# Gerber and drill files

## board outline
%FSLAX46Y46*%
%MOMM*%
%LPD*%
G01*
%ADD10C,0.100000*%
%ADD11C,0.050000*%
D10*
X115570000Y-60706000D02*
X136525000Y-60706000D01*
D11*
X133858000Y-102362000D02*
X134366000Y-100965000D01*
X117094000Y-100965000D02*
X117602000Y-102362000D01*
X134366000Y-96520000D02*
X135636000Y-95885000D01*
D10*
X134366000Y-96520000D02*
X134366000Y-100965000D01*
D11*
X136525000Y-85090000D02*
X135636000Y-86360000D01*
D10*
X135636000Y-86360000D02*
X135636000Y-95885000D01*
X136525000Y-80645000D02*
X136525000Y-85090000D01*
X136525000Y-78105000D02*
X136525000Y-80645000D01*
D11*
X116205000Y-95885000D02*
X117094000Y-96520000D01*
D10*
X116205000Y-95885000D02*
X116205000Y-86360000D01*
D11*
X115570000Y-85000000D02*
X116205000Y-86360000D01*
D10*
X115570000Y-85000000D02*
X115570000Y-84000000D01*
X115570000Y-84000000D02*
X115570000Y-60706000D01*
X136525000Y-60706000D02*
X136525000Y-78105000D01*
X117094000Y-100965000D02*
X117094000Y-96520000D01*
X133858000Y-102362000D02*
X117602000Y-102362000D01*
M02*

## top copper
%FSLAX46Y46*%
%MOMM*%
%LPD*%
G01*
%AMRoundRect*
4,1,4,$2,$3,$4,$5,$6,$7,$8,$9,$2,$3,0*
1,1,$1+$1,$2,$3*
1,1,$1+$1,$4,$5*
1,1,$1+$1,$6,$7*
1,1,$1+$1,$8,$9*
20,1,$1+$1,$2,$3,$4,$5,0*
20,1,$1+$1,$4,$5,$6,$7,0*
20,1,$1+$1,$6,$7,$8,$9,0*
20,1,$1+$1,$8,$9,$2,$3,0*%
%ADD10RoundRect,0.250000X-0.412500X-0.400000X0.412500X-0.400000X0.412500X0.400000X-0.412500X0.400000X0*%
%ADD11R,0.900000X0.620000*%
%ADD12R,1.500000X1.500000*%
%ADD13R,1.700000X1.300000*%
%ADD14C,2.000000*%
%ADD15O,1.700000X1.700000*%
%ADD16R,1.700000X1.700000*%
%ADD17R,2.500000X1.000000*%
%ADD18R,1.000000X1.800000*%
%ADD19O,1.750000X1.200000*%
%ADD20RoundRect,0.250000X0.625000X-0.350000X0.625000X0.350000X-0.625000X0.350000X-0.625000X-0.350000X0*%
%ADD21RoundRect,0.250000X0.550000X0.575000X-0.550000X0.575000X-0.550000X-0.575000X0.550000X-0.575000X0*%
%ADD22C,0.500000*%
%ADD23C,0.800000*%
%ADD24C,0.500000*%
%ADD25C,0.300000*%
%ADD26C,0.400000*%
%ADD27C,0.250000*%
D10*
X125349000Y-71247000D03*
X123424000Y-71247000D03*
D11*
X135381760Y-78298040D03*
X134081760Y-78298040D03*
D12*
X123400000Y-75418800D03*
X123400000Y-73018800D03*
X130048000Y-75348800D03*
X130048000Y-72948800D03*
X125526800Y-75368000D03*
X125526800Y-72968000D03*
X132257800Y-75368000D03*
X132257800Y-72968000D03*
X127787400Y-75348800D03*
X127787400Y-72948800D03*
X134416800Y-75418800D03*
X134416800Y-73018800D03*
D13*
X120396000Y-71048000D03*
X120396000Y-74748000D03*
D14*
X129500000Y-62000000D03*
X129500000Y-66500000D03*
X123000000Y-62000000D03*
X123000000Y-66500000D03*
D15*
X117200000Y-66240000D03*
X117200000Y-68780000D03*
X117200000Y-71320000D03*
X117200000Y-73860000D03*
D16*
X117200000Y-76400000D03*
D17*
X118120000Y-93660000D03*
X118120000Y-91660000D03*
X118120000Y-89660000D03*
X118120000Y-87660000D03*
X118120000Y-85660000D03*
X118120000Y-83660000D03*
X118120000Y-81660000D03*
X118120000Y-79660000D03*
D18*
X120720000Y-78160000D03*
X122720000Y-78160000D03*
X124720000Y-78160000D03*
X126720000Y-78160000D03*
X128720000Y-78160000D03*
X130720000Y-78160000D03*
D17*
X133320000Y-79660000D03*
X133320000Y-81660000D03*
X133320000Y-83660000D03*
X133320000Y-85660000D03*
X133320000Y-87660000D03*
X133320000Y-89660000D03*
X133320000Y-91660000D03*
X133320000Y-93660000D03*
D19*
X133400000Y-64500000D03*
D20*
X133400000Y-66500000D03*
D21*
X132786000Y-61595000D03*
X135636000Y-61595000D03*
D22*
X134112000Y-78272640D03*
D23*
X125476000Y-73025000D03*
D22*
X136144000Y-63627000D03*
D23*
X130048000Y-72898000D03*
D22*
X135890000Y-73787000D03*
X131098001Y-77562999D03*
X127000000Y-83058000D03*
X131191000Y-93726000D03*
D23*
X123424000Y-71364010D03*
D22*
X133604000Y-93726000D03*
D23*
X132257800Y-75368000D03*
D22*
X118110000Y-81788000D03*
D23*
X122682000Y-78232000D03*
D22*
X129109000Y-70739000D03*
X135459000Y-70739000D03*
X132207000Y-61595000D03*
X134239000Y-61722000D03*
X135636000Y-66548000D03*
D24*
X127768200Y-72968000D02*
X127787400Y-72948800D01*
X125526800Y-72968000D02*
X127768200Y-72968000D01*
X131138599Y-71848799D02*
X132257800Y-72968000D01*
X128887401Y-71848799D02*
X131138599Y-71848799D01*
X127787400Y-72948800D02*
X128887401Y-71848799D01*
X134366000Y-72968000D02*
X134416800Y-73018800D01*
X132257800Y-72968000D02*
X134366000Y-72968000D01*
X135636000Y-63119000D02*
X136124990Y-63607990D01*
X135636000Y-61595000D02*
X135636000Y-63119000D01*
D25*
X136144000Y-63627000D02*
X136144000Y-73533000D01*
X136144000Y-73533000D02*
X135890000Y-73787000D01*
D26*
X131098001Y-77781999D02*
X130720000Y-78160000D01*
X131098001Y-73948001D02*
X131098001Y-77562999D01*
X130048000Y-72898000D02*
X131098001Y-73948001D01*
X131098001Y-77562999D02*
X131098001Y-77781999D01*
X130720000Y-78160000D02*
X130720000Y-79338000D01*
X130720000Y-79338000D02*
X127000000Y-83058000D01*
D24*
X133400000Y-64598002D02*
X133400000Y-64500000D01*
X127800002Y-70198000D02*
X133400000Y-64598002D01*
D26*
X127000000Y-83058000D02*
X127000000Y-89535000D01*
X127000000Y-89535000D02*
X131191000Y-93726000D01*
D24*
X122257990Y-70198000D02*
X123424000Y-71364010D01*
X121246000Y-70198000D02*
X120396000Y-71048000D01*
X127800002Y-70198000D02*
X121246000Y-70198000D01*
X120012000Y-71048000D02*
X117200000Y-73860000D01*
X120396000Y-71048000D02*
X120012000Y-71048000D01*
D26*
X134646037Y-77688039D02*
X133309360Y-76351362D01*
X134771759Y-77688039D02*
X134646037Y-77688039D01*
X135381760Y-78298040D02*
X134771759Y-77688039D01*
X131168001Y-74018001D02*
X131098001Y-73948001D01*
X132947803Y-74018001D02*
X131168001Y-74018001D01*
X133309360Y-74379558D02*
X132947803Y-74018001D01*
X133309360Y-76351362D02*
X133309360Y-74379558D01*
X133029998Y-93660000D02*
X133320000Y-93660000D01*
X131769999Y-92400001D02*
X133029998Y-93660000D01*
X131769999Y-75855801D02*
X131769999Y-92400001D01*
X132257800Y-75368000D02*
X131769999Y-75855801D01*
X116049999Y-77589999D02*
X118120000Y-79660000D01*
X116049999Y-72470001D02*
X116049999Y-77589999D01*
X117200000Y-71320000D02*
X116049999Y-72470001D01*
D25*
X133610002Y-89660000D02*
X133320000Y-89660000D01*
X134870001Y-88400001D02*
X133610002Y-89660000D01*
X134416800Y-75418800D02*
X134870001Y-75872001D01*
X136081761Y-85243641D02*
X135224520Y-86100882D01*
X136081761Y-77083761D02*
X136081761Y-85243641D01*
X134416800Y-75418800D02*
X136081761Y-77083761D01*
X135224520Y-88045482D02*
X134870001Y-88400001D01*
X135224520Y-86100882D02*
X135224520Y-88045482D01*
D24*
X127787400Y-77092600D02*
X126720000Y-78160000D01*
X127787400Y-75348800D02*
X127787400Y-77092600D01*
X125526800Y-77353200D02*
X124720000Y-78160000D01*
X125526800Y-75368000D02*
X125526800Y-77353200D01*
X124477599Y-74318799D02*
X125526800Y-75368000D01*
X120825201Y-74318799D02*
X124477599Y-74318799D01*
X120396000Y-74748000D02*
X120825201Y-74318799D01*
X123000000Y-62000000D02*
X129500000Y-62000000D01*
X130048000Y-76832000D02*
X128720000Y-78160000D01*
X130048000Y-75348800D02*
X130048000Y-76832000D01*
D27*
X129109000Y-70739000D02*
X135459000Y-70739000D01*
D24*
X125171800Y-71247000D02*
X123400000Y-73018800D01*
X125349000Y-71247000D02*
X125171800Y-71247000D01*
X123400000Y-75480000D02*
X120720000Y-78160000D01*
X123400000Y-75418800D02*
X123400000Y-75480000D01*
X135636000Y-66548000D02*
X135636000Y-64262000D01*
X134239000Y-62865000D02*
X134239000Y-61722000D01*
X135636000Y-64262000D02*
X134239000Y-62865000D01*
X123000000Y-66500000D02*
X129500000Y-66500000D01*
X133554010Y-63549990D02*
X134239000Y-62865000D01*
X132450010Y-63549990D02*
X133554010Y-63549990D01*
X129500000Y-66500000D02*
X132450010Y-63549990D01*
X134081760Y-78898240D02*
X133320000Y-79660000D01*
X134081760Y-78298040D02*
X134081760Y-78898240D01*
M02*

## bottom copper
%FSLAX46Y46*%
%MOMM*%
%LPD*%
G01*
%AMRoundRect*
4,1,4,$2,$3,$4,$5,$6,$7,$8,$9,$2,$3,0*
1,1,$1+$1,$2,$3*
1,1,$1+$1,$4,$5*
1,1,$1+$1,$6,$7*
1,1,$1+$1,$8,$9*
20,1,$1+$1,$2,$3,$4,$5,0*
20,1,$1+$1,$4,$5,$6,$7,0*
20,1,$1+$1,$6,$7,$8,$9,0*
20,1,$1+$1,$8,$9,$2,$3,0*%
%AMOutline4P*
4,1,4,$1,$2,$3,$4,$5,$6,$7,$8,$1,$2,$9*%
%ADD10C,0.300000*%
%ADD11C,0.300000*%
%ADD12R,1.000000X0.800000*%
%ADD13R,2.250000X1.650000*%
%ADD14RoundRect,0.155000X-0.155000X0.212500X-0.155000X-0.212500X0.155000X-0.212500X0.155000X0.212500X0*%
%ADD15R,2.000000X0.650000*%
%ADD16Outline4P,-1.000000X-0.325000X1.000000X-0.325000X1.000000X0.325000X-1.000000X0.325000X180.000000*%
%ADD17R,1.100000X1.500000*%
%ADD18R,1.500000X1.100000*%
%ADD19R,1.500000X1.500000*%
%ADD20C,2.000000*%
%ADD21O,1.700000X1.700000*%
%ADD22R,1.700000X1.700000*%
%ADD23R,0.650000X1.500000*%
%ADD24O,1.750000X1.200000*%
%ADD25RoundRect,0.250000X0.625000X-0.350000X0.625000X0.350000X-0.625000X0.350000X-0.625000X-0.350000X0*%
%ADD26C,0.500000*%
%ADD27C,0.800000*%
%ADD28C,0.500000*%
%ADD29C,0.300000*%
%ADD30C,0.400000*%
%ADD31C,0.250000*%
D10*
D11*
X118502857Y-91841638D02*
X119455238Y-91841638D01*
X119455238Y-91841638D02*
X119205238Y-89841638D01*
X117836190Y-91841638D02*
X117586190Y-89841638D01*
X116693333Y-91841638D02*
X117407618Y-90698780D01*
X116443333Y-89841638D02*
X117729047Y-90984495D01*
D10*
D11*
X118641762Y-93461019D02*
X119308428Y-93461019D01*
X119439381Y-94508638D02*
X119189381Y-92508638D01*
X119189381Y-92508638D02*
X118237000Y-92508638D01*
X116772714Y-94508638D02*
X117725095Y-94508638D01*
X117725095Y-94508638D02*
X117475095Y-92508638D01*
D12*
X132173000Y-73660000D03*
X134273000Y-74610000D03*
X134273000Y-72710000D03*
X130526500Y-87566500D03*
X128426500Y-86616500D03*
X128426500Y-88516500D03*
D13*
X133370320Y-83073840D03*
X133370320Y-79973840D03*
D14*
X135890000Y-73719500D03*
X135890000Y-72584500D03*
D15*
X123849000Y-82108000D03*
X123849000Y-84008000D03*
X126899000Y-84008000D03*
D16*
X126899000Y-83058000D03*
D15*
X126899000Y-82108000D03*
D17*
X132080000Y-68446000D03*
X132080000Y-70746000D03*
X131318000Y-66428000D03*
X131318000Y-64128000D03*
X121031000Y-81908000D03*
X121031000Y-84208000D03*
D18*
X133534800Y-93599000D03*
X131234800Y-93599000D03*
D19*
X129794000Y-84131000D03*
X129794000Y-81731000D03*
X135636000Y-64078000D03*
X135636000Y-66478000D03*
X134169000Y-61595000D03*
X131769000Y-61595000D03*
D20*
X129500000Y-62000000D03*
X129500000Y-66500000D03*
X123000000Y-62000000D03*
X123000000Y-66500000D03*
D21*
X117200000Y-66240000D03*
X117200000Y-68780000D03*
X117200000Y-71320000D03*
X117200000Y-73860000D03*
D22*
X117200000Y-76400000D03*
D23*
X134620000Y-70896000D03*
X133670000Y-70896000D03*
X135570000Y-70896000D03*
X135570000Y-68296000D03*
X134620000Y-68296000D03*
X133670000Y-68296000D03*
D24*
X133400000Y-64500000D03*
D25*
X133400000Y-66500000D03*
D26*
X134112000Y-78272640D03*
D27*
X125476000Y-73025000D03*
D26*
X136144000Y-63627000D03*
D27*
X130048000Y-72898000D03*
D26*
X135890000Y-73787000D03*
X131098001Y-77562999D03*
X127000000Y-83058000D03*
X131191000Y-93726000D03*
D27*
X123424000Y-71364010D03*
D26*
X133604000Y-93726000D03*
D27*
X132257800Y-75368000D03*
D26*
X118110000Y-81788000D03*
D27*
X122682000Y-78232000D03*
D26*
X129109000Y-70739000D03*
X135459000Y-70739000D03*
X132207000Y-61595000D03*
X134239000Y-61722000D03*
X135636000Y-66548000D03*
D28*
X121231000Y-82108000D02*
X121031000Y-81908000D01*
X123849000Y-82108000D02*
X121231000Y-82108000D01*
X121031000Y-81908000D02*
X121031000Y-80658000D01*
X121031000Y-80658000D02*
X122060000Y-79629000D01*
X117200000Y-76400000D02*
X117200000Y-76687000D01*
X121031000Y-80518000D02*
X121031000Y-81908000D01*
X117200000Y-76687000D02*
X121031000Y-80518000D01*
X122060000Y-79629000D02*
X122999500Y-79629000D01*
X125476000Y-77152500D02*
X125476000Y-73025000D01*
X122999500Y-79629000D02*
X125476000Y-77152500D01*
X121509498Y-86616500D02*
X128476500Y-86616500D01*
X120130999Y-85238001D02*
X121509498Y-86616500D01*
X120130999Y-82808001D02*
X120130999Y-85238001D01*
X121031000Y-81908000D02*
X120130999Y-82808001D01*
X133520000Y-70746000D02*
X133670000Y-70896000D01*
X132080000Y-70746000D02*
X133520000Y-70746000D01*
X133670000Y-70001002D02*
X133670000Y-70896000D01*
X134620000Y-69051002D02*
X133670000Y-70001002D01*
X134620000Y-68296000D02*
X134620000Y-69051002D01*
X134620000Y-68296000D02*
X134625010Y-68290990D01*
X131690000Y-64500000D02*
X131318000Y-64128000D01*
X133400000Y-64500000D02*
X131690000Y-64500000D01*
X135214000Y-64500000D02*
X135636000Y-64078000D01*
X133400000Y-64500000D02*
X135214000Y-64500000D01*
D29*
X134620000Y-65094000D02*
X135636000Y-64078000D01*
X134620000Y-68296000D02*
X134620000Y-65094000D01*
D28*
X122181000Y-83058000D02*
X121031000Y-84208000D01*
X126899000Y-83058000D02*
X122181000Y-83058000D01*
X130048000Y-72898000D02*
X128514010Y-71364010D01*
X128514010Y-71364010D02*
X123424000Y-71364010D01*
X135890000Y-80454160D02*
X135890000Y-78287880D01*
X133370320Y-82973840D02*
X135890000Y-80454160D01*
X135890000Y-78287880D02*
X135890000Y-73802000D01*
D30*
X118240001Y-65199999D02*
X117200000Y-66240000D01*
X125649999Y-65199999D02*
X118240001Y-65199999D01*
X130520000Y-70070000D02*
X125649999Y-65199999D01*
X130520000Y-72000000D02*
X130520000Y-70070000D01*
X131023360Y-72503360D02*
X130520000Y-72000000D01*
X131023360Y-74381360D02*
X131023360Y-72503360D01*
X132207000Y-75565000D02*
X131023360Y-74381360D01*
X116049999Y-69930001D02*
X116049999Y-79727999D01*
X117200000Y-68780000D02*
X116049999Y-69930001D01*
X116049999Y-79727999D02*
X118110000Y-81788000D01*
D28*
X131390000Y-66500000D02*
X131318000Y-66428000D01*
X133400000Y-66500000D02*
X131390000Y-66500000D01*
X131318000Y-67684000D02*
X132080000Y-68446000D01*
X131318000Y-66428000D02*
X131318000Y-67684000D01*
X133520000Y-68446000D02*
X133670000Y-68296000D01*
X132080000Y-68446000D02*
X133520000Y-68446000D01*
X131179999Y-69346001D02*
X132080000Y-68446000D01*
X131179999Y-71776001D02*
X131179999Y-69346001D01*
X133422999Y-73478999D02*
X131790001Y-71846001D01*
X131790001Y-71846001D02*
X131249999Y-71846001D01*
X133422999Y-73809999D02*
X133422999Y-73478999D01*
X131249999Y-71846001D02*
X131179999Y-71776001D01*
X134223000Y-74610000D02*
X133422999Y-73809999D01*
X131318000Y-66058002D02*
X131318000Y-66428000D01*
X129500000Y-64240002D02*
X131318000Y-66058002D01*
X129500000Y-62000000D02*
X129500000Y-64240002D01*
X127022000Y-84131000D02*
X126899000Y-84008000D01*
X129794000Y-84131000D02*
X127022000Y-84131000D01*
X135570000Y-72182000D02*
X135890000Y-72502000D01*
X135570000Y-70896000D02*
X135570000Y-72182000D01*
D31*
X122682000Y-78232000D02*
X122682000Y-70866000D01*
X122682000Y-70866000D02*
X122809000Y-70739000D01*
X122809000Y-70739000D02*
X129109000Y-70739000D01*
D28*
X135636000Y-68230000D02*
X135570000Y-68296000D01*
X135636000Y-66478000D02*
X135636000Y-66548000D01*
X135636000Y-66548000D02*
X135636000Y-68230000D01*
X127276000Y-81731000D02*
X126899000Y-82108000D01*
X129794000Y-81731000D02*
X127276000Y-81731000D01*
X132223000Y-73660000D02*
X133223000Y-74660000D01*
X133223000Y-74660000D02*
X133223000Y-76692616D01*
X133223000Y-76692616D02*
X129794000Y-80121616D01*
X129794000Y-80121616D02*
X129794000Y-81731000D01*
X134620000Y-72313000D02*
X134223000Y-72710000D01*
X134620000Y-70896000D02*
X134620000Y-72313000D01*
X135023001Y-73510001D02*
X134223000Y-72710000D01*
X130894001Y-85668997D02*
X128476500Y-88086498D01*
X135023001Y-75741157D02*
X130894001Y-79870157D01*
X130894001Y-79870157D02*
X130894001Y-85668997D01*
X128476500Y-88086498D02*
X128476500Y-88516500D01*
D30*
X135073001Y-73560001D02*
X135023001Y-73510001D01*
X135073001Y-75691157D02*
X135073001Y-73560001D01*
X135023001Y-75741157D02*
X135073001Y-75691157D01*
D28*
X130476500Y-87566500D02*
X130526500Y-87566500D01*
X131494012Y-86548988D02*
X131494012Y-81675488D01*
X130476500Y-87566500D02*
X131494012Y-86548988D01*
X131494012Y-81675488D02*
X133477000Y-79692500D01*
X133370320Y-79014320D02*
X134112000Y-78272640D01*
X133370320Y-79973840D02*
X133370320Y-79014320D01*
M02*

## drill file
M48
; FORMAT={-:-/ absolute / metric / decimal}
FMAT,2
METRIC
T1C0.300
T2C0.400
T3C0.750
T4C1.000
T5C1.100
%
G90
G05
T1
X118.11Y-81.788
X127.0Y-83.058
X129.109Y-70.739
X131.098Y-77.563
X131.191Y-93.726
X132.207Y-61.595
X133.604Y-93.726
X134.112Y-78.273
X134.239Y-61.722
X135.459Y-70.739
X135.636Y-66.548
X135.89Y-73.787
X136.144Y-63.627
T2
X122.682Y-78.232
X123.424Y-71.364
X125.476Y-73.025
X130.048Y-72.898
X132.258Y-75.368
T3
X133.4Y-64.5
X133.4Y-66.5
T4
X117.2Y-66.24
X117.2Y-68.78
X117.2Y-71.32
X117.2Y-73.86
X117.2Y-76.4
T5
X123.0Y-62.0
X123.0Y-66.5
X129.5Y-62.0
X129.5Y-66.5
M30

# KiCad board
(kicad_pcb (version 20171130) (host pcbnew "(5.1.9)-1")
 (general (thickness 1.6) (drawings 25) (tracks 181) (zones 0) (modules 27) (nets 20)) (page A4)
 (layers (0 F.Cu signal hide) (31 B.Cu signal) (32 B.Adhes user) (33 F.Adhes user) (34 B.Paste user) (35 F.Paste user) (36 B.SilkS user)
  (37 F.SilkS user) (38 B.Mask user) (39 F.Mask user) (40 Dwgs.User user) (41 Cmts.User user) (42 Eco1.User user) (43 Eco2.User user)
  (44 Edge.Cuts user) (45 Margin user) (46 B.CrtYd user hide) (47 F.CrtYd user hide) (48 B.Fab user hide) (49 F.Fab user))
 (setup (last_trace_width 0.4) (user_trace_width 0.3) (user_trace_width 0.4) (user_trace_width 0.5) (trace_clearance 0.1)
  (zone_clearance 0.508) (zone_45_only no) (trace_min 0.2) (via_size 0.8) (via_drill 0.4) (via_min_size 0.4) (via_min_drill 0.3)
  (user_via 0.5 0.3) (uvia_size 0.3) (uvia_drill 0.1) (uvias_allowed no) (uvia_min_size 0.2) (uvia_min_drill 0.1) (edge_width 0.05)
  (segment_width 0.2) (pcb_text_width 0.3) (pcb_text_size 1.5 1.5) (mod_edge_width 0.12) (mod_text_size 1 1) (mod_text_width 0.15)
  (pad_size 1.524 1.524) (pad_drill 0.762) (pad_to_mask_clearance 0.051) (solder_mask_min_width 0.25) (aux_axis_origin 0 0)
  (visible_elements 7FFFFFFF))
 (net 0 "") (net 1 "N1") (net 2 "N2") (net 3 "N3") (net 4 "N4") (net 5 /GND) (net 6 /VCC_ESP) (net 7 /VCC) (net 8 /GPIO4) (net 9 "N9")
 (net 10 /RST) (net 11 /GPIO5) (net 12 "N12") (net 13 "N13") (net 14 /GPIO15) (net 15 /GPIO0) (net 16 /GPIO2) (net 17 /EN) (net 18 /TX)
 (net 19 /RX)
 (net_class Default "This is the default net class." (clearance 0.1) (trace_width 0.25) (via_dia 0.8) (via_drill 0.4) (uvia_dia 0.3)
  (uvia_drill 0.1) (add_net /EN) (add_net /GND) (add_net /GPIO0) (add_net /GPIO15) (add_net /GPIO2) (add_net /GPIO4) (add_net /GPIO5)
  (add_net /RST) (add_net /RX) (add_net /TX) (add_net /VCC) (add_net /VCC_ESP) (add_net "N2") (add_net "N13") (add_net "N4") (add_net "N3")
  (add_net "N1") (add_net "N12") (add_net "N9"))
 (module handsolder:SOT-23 (layer B.Cu) (at 133.223 73.66 180)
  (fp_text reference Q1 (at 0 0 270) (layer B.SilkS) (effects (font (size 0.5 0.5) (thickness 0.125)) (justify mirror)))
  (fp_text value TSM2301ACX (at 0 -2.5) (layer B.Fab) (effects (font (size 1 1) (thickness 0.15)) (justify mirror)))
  (pad 3 smd rect (at 1.05 0 180) (size 1 0.8) (layers B.Cu B.Paste B.Mask) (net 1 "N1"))
  (pad 2 smd rect (at -1.05 -0.95 180) (size 1 0.8) (layers B.Cu B.Paste B.Mask) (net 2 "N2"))
  (pad 1 smd rect (at -1.05 0.95 180) (size 1 0.8) (layers B.Cu B.Paste B.Mask) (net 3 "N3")))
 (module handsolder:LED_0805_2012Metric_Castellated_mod (layer F.Cu) (at 124.3865 71.247)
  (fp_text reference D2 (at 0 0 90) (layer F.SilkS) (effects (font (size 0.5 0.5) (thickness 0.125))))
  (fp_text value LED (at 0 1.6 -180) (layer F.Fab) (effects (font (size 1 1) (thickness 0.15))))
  (pad 2 smd roundrect (at 0.9625 0) (size 1.325 1.3) (layers F.Cu F.Paste F.Mask) (roundrect_rratio 0.1923076923076923) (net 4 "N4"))
  (pad 1 smd roundrect (at -0.9625 0) (size 1.325 1.3) (layers F.Cu F.Paste F.Mask) (roundrect_rratio 0.1923076923076923) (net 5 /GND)))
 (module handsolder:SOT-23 (layer B.Cu) (at 129.4765 87.5665)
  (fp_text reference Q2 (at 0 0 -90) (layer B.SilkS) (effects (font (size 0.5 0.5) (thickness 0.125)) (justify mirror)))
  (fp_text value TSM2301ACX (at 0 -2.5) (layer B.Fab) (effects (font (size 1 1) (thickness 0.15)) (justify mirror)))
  (pad 3 smd rect (at 1.05 0) (size 1 0.8) (layers B.Cu B.Paste B.Mask) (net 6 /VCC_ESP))
  (pad 2 smd rect (at -1.05 -0.95) (size 1 0.8) (layers B.Cu B.Paste B.Mask) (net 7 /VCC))
  (pad 1 smd rect (at -1.05 0.95) (size 1 0.8) (layers B.Cu B.Paste B.Mask) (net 3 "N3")))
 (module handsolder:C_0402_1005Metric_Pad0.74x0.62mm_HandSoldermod (layer F.Cu) (at 134.73176 78.29804)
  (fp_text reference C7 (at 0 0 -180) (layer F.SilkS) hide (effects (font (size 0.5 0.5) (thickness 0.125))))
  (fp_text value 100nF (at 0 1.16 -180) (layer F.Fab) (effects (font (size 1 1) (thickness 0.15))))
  (pad 2 smd rect (at 0.65 0) (size 0.9 0.62) (layers F.Cu F.Paste F.Mask) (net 5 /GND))
  (pad 1 smd rect (at -0.65 0) (size 0.9 0.62) (layers F.Cu F.Paste F.Mask) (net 6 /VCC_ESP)))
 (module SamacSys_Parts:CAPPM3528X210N (layer B.Cu) (at 133.37032 81.52384 270)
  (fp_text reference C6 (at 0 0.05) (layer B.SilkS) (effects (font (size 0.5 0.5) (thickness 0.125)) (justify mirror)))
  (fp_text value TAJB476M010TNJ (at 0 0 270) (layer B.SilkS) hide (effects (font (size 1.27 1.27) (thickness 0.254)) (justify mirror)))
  (pad 2 smd rect (at 1.55 0 270) (size 1.65 2.25) (layers B.Cu B.Paste B.Mask) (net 5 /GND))
  (pad 1 smd rect (at -1.55 0 270) (size 1.65 2.25) (layers B.Cu B.Paste B.Mask) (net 6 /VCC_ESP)))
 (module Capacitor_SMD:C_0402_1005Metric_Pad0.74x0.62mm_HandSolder (layer B.Cu) (at 135.89 73.152 270)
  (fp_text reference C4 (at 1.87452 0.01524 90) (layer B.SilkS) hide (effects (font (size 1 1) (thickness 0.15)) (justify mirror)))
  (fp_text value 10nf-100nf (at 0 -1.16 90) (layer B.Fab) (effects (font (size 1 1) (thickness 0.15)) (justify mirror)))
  (pad 2 smd roundrect (at 0.5675 0 270) (size 0.735 0.62) (layers B.Cu B.Paste B.Mask) (roundrect_rratio 0.25) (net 5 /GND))
  (pad 1 smd roundrect (at -0.5675 0 270) (size 0.735 0.62) (layers B.Cu B.Paste B.Mask) (roundrect_rratio 0.25) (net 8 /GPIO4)))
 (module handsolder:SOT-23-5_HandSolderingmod (layer B.Cu) (at 125.349 83.058 180)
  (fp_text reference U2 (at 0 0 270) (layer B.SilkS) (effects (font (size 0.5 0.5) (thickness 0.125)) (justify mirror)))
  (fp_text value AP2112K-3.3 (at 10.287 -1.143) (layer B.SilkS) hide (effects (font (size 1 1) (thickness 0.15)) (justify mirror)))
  (pad 5 smd rect (at 1.5 0.95 180) (size 2 0.65) (layers B.Cu B.Paste B.Mask) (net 7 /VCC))
  (pad 4 smd rect (at 1.5 -0.95 180) (size 2 0.65) (layers B.Cu B.Paste B.Mask))
  (pad 3 smd rect (at -1.55 -0.95 180) (size 2 0.65) (layers B.Cu B.Paste B.Mask) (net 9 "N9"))
  (pad 2 smd trapezoid (at -1.55 0 180) (size 2 0.65) (layers B.Cu B.Paste B.Mask) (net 5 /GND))
  (pad 1 smd rect (at -1.55 0.95 180) (size 2 0.65) (layers B.Cu B.Paste B.Mask) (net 1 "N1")))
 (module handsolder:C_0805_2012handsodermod (layer B.Cu) (at 132.08 69.596 90)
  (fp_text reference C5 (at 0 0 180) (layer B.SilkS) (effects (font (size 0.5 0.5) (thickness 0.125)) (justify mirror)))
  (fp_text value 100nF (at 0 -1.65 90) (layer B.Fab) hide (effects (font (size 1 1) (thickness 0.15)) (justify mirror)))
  (pad 2 smd rect (at 1.15 0 90) (size 1.5 1.1) (layers B.Cu B.Paste B.Mask) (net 2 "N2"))
  (pad 1 smd rect (at -1.15 0 90) (size 1.5 1.1) (layers B.Cu B.Paste B.Mask) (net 5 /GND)))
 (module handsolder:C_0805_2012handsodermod (layer B.Cu) (at 131.318 65.278 270)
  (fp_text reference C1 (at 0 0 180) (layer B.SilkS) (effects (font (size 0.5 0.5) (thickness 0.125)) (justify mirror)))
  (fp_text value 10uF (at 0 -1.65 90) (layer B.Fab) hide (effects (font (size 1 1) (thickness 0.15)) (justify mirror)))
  (pad 2 smd rect (at 1.15 0 270) (size 1.5 1.1) (layers B.Cu B.Paste B.Mask) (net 2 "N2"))
  (pad 1 smd rect (at -1.15 0 270) (size 1.5 1.1) (layers B.Cu B.Paste B.Mask) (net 5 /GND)))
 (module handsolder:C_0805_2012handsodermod (layer B.Cu) (at 121.031 83.058 90)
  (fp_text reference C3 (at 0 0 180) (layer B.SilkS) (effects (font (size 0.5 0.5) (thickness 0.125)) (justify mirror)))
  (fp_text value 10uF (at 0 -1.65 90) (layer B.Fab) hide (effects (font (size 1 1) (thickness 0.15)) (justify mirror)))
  (pad 2 smd rect (at 1.15 0 90) (size 1.5 1.1) (layers B.Cu B.Paste B.Mask) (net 7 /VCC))
  (pad 1 smd rect (at -1.15 0 90) (size 1.5 1.1) (layers B.Cu B.Paste B.Mask) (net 5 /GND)))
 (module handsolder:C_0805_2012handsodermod (layer B.Cu) (at 132.3848 93.599)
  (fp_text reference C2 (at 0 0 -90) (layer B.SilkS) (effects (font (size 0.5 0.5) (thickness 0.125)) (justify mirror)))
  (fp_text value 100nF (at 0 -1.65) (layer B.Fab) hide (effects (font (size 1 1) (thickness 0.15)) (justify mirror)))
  (pad 2 smd rect (at 1.15 0) (size 1.5 1.1) (layers B.Cu B.Paste B.Mask) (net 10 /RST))
  (pad 1 smd rect (at -1.15 0) (size 1.5 1.1) (layers B.Cu B.Paste B.Mask) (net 5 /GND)))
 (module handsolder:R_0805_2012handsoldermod (layer F.Cu) (at 123.4 74.2188 270)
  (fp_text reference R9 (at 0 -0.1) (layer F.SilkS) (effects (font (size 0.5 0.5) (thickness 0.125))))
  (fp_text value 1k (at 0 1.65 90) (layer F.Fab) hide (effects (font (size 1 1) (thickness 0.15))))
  (pad 2 smd rect (at 1.2 0 270) (size 1.5 1.5) (layers F.Cu F.Paste F.Mask) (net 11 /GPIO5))
  (pad 1 smd rect (at -1.2 0 270) (size 1.5 1.5) (layers F.Cu F.Paste F.Mask) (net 4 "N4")))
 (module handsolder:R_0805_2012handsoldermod (layer B.Cu) (at 129.794 82.931 270)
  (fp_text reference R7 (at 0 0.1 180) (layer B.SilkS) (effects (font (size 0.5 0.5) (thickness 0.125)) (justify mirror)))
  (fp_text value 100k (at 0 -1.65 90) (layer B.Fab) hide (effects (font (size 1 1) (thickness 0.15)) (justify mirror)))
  (pad 2 smd rect (at 1.2 0 270) (size 1.5 1.5) (layers B.Cu B.Paste B.Mask) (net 9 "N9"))
  (pad 1 smd rect (at -1.2 0 270) (size 1.5 1.5) (layers B.Cu B.Paste B.Mask) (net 1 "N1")))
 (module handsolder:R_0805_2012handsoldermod (layer B.Cu) (at 135.636 65.278 90)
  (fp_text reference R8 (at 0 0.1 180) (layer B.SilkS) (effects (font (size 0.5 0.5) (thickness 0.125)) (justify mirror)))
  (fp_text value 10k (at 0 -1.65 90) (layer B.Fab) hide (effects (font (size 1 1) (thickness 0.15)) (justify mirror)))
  (pad 2 smd rect (at 1.2 0 90) (size 1.5 1.5) (layers B.Cu B.Paste B.Mask) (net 5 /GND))
  (pad 1 smd rect (at -1.2 0 90) (size 1.5 1.5) (layers B.Cu B.Paste B.Mask) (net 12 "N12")))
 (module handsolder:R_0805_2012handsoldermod (layer B.Cu) (at 132.969 61.595)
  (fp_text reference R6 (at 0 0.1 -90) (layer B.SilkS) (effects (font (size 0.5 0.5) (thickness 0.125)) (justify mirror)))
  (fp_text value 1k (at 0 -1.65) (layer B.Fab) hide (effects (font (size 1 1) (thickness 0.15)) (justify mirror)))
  (pad 2 smd rect (at 1.2 0) (size 1.5 1.5) (layers B.Cu B.Paste B.Mask) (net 12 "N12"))
  (pad 1 smd rect (at -1.2 0) (size 1.5 1.5) (layers B.Cu B.Paste B.Mask) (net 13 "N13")))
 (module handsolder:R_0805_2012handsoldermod (layer F.Cu) (at 130.048 74.1488 270)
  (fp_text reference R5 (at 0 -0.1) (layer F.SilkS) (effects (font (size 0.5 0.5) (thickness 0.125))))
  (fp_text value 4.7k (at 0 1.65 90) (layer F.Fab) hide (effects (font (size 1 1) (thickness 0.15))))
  (pad 2 smd rect (at 1.2 0 270) (size 1.5 1.5) (layers F.Cu F.Paste F.Mask) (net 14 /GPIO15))
  (pad 1 smd rect (at -1.2 0 270) (size 1.5 1.5) (layers F.Cu F.Paste F.Mask) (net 5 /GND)))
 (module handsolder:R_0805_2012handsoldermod (layer F.Cu) (at 125.5268 74.168 270)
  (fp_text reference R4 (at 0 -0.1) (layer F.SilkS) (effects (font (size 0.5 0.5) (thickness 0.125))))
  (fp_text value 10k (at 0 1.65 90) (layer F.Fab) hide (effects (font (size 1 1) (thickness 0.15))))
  (pad 2 smd rect (at 1.2 0 270) (size 1.5 1.5) (layers F.Cu F.Paste F.Mask) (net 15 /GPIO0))
  (pad 1 smd rect (at -1.2 0 270) (size 1.5 1.5) (layers F.Cu F.Paste F.Mask) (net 7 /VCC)))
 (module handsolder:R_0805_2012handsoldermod (layer F.Cu) (at 132.2578 74.168 270)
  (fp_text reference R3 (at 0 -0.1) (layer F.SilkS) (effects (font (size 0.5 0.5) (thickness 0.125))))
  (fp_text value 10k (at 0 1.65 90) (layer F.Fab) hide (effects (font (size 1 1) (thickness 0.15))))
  (pad 2 smd rect (at 1.2 0 270) (size 1.5 1.5) (layers F.Cu F.Paste F.Mask) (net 10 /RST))
  (pad 1 smd rect (at -1.2 0 270) (size 1.5 1.5) (layers F.Cu F.Paste F.Mask) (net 7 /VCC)))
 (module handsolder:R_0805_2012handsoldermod (layer F.Cu) (at 127.7874 74.1488 270)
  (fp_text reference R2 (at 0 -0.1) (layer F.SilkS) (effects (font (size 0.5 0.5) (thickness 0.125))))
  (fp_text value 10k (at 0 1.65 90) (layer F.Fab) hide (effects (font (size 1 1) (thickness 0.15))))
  (pad 2 smd rect (at 1.2 0 270) (size 1.5 1.5) (layers F.Cu F.Paste F.Mask) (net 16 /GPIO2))
  (pad 1 smd rect (at -1.2 0 270) (size 1.5 1.5) (layers F.Cu F.Paste F.Mask) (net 7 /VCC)))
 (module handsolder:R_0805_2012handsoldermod (layer F.Cu) (at 134.4168 74.2188 270)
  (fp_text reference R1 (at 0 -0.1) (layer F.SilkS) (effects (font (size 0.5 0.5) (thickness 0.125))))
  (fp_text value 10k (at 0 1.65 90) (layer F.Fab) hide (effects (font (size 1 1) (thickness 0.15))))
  (pad 2 smd rect (at 1.2 0 270) (size 1.5 1.5) (layers F.Cu F.Paste F.Mask) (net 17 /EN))
  (pad 1 smd rect (at -1.2 0 270) (size 1.5 1.5) (layers F.Cu F.Paste F.Mask) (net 7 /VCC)))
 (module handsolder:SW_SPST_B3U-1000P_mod (layer F.Cu) (at 120.396 72.898 90)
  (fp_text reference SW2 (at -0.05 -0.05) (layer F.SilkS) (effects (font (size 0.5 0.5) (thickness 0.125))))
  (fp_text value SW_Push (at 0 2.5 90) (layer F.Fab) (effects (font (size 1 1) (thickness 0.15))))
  (pad 2 smd rect (at 1.85 0 90) (size 1.3 1.7) (layers F.Cu F.Paste F.Mask) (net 5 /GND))
  (pad 1 smd rect (at -1.85 0 90) (size 1.3 1.7) (layers F.Cu F.Paste F.Mask) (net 15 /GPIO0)))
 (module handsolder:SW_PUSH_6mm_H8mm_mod (layer F.Cu) (at 123 62)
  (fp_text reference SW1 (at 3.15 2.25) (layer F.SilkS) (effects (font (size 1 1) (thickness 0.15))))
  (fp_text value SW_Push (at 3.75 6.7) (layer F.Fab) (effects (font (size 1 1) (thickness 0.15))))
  (pad 1 thru_hole circle (at 6.5 0 90) (size 2 2) (drill 1.1) (layers *.Cu *.Mask) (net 2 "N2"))
  (pad 2 thru_hole circle (at 6.5 4.5 90) (size 2 2) (drill 1.1) (layers *.Cu *.Mask) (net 12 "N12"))
  (pad 1 thru_hole circle (at 0 0 90) (size 2 2) (drill 1.1) (layers *.Cu *.Mask) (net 2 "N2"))
  (pad 2 thru_hole circle (at 0 4.5 90) (size 2 2) (drill 1.1) (layers *.Cu *.Mask) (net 12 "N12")))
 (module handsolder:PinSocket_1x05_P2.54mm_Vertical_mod (layer F.Cu) (at 117.2 76.4 180)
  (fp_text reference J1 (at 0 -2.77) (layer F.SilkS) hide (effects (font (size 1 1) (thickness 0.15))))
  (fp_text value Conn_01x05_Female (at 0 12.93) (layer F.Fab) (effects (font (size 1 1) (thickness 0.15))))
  (pad 5 thru_hole oval (at 0 10.16 180) (size 1.7 1.7) (drill 1) (layers *.Cu *.Mask) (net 10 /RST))
  (pad 4 thru_hole oval (at 0 7.62 180) (size 1.7 1.7) (drill 1) (layers *.Cu *.Mask) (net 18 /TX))
  (pad 3 thru_hole oval (at 0 5.08 180) (size 1.7 1.7) (drill 1) (layers *.Cu *.Mask) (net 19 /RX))
  (pad 2 thru_hole oval (at 0 2.54 180) (size 1.7 1.7) (drill 1) (layers *.Cu *.Mask) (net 5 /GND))
  (pad 1 thru_hole rect (at 0 0 180) (size 1.7 1.7) (drill 1) (layers *.Cu *.Mask) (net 7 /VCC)))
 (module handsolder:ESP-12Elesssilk (layer F.Cu) (at 125.72 90.16 180)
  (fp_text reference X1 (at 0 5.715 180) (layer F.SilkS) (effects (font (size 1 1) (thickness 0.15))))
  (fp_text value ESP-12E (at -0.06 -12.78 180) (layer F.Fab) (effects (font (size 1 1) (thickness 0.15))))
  (pad 22 smd rect (at 7.6 -3.5 180) (size 2.5 1) (layers F.Cu F.Paste F.Mask))
  (pad 21 smd rect (at 7.6 -1.5 180) (size 2.5 1) (layers F.Cu F.Paste F.Mask))
  (pad 20 smd rect (at 7.6 0.5 180) (size 2.5 1) (layers F.Cu F.Paste F.Mask))
  (pad 19 smd rect (at 7.6 2.5 180) (size 2.5 1) (layers F.Cu F.Paste F.Mask))
  (pad 18 smd rect (at 7.6 4.5 180) (size 2.5 1) (layers F.Cu F.Paste F.Mask))
  (pad 17 smd rect (at 7.6 6.5 180) (size 2.5 1) (layers F.Cu F.Paste F.Mask))
  (pad 16 smd rect (at 7.6 8.5 180) (size 2.5 1) (layers F.Cu F.Paste F.Mask) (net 18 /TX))
  (pad 15 smd rect (at 7.6 10.5 180) (size 2.5 1) (layers F.Cu F.Paste F.Mask) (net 19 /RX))
  (pad 14 smd rect (at 5 12 180) (size 1 1.8) (layers F.Cu F.Paste F.Mask) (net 11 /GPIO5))
  (pad 13 smd rect (at 3 12 180) (size 1 1.8) (layers F.Cu F.Paste F.Mask) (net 8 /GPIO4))
  (pad 12 smd rect (at 1 12 180) (size 1 1.8) (layers F.Cu F.Paste F.Mask) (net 15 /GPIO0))
  (pad 11 smd rect (at -1 12 180) (size 1 1.8) (layers F.Cu F.Paste F.Mask) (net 16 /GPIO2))
  (pad 10 smd rect (at -3 12 180) (size 1 1.8) (layers F.Cu F.Paste F.Mask) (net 14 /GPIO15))
  (pad 9 smd rect (at -5 12 180) (size 1 1.8) (layers F.Cu F.Paste F.Mask) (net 5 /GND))
  (pad 8 smd rect (at -7.6 10.5 180) (size 2.5 1) (layers F.Cu F.Paste F.Mask) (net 6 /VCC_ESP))
  (pad 7 smd rect (at -7.6 8.5 180) (size 2.5 1) (layers F.Cu F.Paste F.Mask))
  (pad 6 smd rect (at -7.6 6.5 180) (size 2.5 1) (layers F.Cu F.Paste F.Mask))
  (pad 5 smd rect (at -7.6 4.5 180) (size 2.5 1) (layers F.Cu F.Paste F.Mask))
  (pad 4 smd rect (at -7.6 2.5 180) (size 2.5 1) (layers F.Cu F.Paste F.Mask))
  (pad 3 smd rect (at -7.6 0.5 180) (size 2.5 1) (layers F.Cu F.Paste F.Mask) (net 17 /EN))
  (pad 2 smd rect (at -7.6 -1.5 180) (size 2.5 1) (layers F.Cu F.Paste F.Mask))
  (pad 1 smd rect (at -7.6 -3.5 180) (size 2.5 1) (layers F.Cu F.Paste F.Mask) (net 10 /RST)))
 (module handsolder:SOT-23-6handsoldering (layer B.Cu) (at 134.62 69.596 270)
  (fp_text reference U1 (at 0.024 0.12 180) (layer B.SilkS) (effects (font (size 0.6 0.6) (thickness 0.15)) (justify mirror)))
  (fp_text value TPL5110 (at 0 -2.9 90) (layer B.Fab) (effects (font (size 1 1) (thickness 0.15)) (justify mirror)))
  (pad 5 smd rect (at 1.3 0 270) (size 1.5 0.65) (layers B.Cu B.Paste B.Mask) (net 3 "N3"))
  (pad 6 smd rect (at 1.3 0.95 270) (size 1.5 0.65) (layers B.Cu B.Paste B.Mask) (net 5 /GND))
  (pad 4 smd rect (at 1.3 -0.95 270) (size 1.5 0.65) (layers B.Cu B.Paste B.Mask) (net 8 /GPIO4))
  (pad 3 smd rect (at -1.3 -0.95 270) (size 1.5 0.65) (layers B.Cu B.Paste B.Mask) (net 12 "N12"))
  (pad 2 smd rect (at -1.3 0 270) (size 1.5 0.65) (layers B.Cu B.Paste B.Mask) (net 5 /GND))
  (pad 1 smd rect (at -1.3 0.95 270) (size 1.5 0.65) (layers B.Cu B.Paste B.Mask) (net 2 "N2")))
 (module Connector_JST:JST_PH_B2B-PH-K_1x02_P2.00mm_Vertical (layer F.Cu) (at 133.4 66.5 90)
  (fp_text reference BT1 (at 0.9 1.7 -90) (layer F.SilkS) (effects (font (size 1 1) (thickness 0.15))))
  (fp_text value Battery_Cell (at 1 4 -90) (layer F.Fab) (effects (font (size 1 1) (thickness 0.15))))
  (pad 2 thru_hole oval (at 2 0 90) (size 1.2 1.75) (drill 0.75) (layers *.Cu *.Mask) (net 5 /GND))
  (pad 1 thru_hole roundrect (at 0 0 90) (size 1.2 1.75) (drill 0.75) (layers *.Cu *.Mask) (roundrect_rratio 0.208333) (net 2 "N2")))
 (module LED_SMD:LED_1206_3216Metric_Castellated (layer F.Cu) (at 134.211 61.595 180)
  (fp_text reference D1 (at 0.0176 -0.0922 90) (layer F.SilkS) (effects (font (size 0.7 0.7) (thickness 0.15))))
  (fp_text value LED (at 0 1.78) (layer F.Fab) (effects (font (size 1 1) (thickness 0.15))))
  (pad 2 smd roundrect (at 1.425 0 180) (size 1.6 1.65) (layers F.Cu F.Paste F.Mask) (roundrect_rratio 0.15625) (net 13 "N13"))
  (pad 1 smd roundrect (at -1.425 0 180) (size 1.6 1.65) (layers F.Cu F.Paste F.Mask) (roundrect_rratio 0.15625) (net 5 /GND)))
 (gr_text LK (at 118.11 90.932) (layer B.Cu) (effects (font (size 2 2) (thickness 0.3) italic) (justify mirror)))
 (gr_line (start 115.57 60.706) (end 136.525 60.706) (layer Edge.Cuts) (width 0.1))
 (gr_line (start 133.858 102.362) (end 134.366 100.965) (layer Edge.Cuts) (width 0.05))
 (gr_line (start 117.094 100.965) (end 117.602 102.362) (layer Edge.Cuts) (width 0.05))
 (gr_line (start 134.366 96.52) (end 135.636 95.885) (layer Edge.Cuts) (width 0.05))
 (gr_line (start 134.366 96.52) (end 134.366 100.965) (layer Edge.Cuts) (width 0.1))
 (gr_line (start 136.525 85.09) (end 135.636 86.36) (layer Edge.Cuts) (width 0.05))
 (gr_line (start 135.636 86.36) (end 135.636 95.885) (layer Edge.Cuts) (width 0.1))
 (gr_line (start 136.525 80.645) (end 136.525 85.09) (layer Edge.Cuts) (width 0.1))
 (gr_line (start 136.525 78.105) (end 136.525 80.645) (layer Edge.Cuts) (width 0.1))
 (gr_line (start 116.205 95.885) (end 117.094 96.52) (layer Edge.Cuts) (width 0.05))
 (gr_line (start 116.205 95.885) (end 116.205 86.36) (layer Edge.Cuts) (width 0.1))
 (gr_line (start 115.57 85) (end 116.205 86.36) (layer Edge.Cuts) (width 0.05))
 (gr_line (start 115.57 85) (end 115.57 84) (layer Edge.Cuts) (width 0.1))
 (gr_line (start 115.57 84) (end 115.57 60.706) (layer Edge.Cuts) (width 0.1))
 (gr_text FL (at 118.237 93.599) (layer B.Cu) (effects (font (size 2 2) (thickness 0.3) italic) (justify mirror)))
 (gr_line (start 136.525 60.706) (end 136.525 78.105) (layer Edge.Cuts) (width 0.1))
 (gr_line (start 117.094 100.965) (end 117.094 96.52) (layer Edge.Cuts) (width 0.1))
 (gr_line (start 133.858 102.362) (end 117.602 102.362) (layer Edge.Cuts) (width 0.1))
 (via (at 134.112 78.27264) (size 0.5) (drill 0.3) (layers F.Cu B.Cu) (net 6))
 (via (at 125.476 73.025) (size 0.8) (drill 0.4) (layers F.Cu B.Cu) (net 7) (status 30))
 (segment (start 121.231 82.108) (end 121.031 81.908) (width 0.5) (layer B.Cu) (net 7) (status 30))
 (segment (start 123.849 82.108) (end 121.231 82.108) (width 0.5) (layer B.Cu) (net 7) (status 30))
 (segment (start 121.031 81.908) (end 121.031 80.658) (width 0.5) (layer B.Cu) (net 7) (status 10))
 (segment (start 121.031 80.658) (end 122.06 79.629) (width 0.5) (layer B.Cu) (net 7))
 (segment (start 127.7682 72.968) (end 127.7874 72.9488) (width 0.5) (layer F.Cu) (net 7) (status 30))
 (segment (start 125.5268 72.968) (end 127.7682 72.968) (width 0.5) (layer F.Cu) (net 7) (status 30))
 (segment (start 131.138599 71.848799) (end 132.2578 72.968) (width 0.5) (layer F.Cu) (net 7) (status 20))
 (segment (start 128.887401 71.848799) (end 131.138599 71.848799) (width 0.5) (layer F.Cu) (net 7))
 (segment (start 127.7874 72.9488) (end 128.887401 71.848799) (width 0.5) (layer F.Cu) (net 7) (status 10))
 (segment (start 134.366 72.968) (end 134.4168 73.0188) (width 0.5) (layer F.Cu) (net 7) (status 30))
 (segment (start 132.2578 72.968) (end 134.366 72.968) (width 0.5) (layer F.Cu) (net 7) (status 30))
 (segment (start 117.2 76.4) (end 117.2 76.687) (width 0.5) (layer B.Cu) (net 7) (status 30))
 (segment (start 121.031 80.518) (end 121.031 81.908) (width 0.5) (layer B.Cu) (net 7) (status 20))
 (segment (start 117.2 76.687) (end 121.031 80.518) (width 0.5) (layer B.Cu) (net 7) (status 10))
 (segment (start 122.06 79.629) (end 122.9995 79.629) (width 0.5) (layer B.Cu) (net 7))
 (segment (start 125.476 77.1525) (end 125.476 73.025) (width 0.5) (layer B.Cu) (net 7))
 (segment (start 122.9995 79.629) (end 125.476 77.1525) (width 0.5) (layer B.Cu) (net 7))
 (segment (start 121.509498 86.6165) (end 128.4765 86.6165) (width 0.5) (layer B.Cu) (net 7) (status 20))
 (segment (start 120.130999 85.238001) (end 121.509498 86.6165) (width 0.5) (layer B.Cu) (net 7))
 (segment (start 120.130999 82.808001) (end 120.130999 85.238001) (width 0.5) (layer B.Cu) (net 7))
 (segment (start 121.031 81.908) (end 120.130999 82.808001) (width 0.5) (layer B.Cu) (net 7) (status 10))
 (via (at 136.144 63.627) (size 0.5) (drill 0.3) (layers F.Cu B.Cu) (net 5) (status 30))
 (segment (start 133.52 70.746) (end 133.67 70.896) (width 0.5) (layer B.Cu) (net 5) (status 30))
 (segment (start 132.08 70.746) (end 133.52 70.746) (width 0.5) (layer B.Cu) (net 5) (status 30))
 (segment (start 133.67 70.001002) (end 133.67 70.896) (width 0.5) (layer B.Cu) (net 5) (status 20))
 (segment (start 134.62 69.051002) (end 133.67 70.001002) (width 0.5) (layer B.Cu) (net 5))
 (segment (start 134.62 68.296) (end 134.62 69.051002) (width 0.5) (layer B.Cu) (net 5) (status 10))
 (segment (start 134.62 68.296) (end 134.62501 68.29099) (width 0.5) (layer B.Cu) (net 5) (status 30))
 (segment (start 131.69 64.5) (end 131.318 64.128) (width 0.5) (layer B.Cu) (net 5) (status 30))
 (segment (start 133.4 64.5) (end 131.69 64.5) (width 0.5) (layer B.Cu) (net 5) (status 30))
 (segment (start 135.214 64.5) (end 135.636 64.078) (width 0.5) (layer B.Cu) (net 5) (status 30))
 (segment (start 133.4 64.5) (end 135.214 64.5) (width 0.5) (layer B.Cu) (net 5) (status 30))
 (segment (start 134.62 65.094) (end 135.636 64.078) (width 0.3) (layer B.Cu) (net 5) (status 20))
 (segment (start 134.62 68.296) (end 134.62 65.094) (width 0.3) (layer B.Cu) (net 5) (status 10))
 (segment (start 122.181 83.058) (end 121.031 84.208) (width 0.5) (layer B.Cu) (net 5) (status 20))
 (segment (start 126.899 83.058) (end 122.181 83.058) (width 0.5) (layer B.Cu) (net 5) (status 10))
 (segment (start 135.636 63.119) (end 136.12499 63.60799) (width 0.5) (layer F.Cu) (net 5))
 (segment (start 135.636 61.595) (end 135.636 63.119) (width 0.5) (layer F.Cu) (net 5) (status 10))
 (via (at 130.048 72.898) (size 0.8) (drill 0.4) (layers F.Cu B.Cu) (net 5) (status 30))
 (segment (start 136.144 63.627) (end 136.144 73.533) (width 0.3) (layer F.Cu) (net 5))
 (segment (start 136.144 73.533) (end 135.89 73.787) (width 0.3) (layer F.Cu) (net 5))
 (via (at 135.89 73.787) (size 0.5) (drill 0.3) (layers F.Cu B.Cu) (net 5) (status 30))
 (segment (start 131.098001 77.781999) (end 130.72 78.16) (width 0.4) (layer F.Cu) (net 5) (status 30))
 (segment (start 131.098001 73.948001) (end 131.098001 77.562999) (width 0.4) (layer F.Cu) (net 5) (status 20))
 (segment (start 130.048 72.898) (end 131.098001 73.948001) (width 0.4) (layer F.Cu) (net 5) (status 10))
 (segment (start 131.098001 77.562999) (end 131.098001 77.781999) (width 0.4) (layer F.Cu) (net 5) (status 30))
 (via (at 131.098001 77.562999) (size 0.5) (drill 0.3) (layers F.Cu B.Cu) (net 5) (status 30))
 (segment (start 130.72 78.16) (end 130.72 79.338) (width 0.4) (layer F.Cu) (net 5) (status 10))
 (segment (start 130.72 79.338) (end 127 83.058) (width 0.4) (layer F.Cu) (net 5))
 (via (at 127 83.058) (size 0.5) (drill 0.3) (layers F.Cu B.Cu) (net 5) (status 30))
 (segment (start 133.4 64.598002) (end 133.4 64.5) (width 0.5) (layer F.Cu) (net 5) (status 30))
 (segment (start 127.800002 70.198) (end 133.4 64.598002) (width 0.5) (layer F.Cu) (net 5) (status 20))
 (via (at 131.191 93.726) (size 0.5) (drill 0.3) (layers F.Cu B.Cu) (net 5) (status 30))
 (segment (start 127 83.058) (end 127 89.535) (width 0.4) (layer F.Cu) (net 5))
 (segment (start 127 89.535) (end 131.191 93.726) (width 0.4) (layer F.Cu) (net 5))
 (via (at 123.424 71.36401) (size 0.8) (drill 0.4) (layers F.Cu B.Cu) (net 5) (status 30))
 (segment (start 122.25799 70.198) (end 123.424 71.36401) (width 0.5) (layer F.Cu) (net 5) (status 20))
 (segment (start 130.048 72.898) (end 128.51401 71.36401) (width 0.5) (layer B.Cu) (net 5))
 (segment (start 128.51401 71.36401) (end 123.424 71.36401) (width 0.5) (layer B.Cu) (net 5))
 (segment (start 121.246 70.198) (end 120.396 71.048) (width 0.5) (layer F.Cu) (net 5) (status 20))
 (segment (start 127.800002 70.198) (end 121.246 70.198) (width 0.5) (layer F.Cu) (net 5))
 (segment (start 120.012 71.048) (end 117.2 73.86) (width 0.5) (layer F.Cu) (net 5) (status 30))
 (segment (start 120.396 71.048) (end 120.012 71.048) (width 0.5) (layer F.Cu) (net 5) (status 30))
 (segment (start 135.89 80.45416) (end 135.89 78.28788) (width 0.5) (layer B.Cu) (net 5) (status 20))
 (segment (start 133.37032 82.97384) (end 135.89 80.45416) (width 0.5) (layer B.Cu) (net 5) (status 10))
 (segment (start 135.89 78.28788) (end 135.89 73.802) (width 0.5) (layer B.Cu) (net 5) (status 20))
 (segment (start 134.646037 77.688039) (end 133.30936 76.351362) (width 0.4) (layer F.Cu) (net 5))
 (segment (start 134.771759 77.688039) (end 134.646037 77.688039) (width 0.4) (layer F.Cu) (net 5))
 (segment (start 135.38176 78.29804) (end 134.771759 77.688039) (width 0.4) (layer F.Cu) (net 5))
 (segment (start 131.168001 74.018001) (end 131.098001 73.948001) (width 0.4) (layer F.Cu) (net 5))
 (segment (start 132.947803 74.018001) (end 131.168001 74.018001) (width 0.4) (layer F.Cu) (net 5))
 (segment (start 133.30936 74.379558) (end 132.947803 74.018001) (width 0.4) (layer F.Cu) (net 5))
 (segment (start 133.30936 76.351362) (end 133.30936 74.379558) (width 0.4) (layer F.Cu) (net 5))
 (via (at 133.604 93.726) (size 0.5) (drill 0.3) (layers F.Cu B.Cu) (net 10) (status 30))
 (segment (start 133.029998 93.66) (end 133.32 93.66) (width 0.4) (layer F.Cu) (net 10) (status 30))
 (segment (start 131.769999 92.400001) (end 133.029998 93.66) (width 0.4) (layer F.Cu) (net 10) (status 20))
 (segment (start 131.769999 75.855801) (end 131.769999 92.400001) (width 0.4) (layer F.Cu) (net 10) (status 10))
 (segment (start 132.2578 75.368) (end 131.769999 75.855801) (width 0.4) (layer F.Cu) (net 10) (status 30))
 (via (at 132.2578 75.368) (size 0.8) (drill 0.4) (layers F.Cu B.Cu) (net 10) (status 30))
 (segment (start 118.240001 65.199999) (end 117.2 66.24) (width 0.4) (layer B.Cu) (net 10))
 (segment (start 125.649999 65.199999) (end 118.240001 65.199999) (width 0.4) (layer B.Cu) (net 10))
 (segment (start 130.52 70.07) (end 125.649999 65.199999) (width 0.4) (layer B.Cu) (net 10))
 (segment (start 130.52 72) (end 130.52 70.07) (width 0.4) (layer B.Cu) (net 10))
 (segment (start 131.02336 72.50336) (end 130.52 72) (width 0.4) (layer B.Cu) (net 10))
 (segment (start 131.02336 74.38136) (end 131.02336 72.50336) (width 0.4) (layer B.Cu) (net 10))
 (segment (start 132.207 75.565) (end 131.02336 74.38136) (width 0.4) (layer B.Cu) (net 10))
 (segment (start 116.049999 77.589999) (end 118.12 79.66) (width 0.4) (layer F.Cu) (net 19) (status 20))
 (segment (start 116.049999 72.470001) (end 116.049999 77.589999) (width 0.4) (layer F.Cu) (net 19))
 (segment (start 117.2 71.32) (end 116.049999 72.470001) (width 0.4) (layer F.Cu) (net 19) (status 10))
 (segment (start 116.049999 69.930001) (end 116.049999 79.727999) (width 0.4) (layer B.Cu) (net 18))
 (segment (start 117.2 68.78) (end 116.049999 69.930001) (width 0.4) (layer B.Cu) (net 18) (status 10))
 (segment (start 116.049999 79.727999) (end 118.11 81.788) (width 0.4) (layer B.Cu) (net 18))
 (via (at 118.11 81.788) (size 0.5) (drill 0.3) (layers F.Cu B.Cu) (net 18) (status 30))
 (segment (start 133.610002 89.66) (end 133.32 89.66) (width 0.3) (layer F.Cu) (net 17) (status 30))
 (segment (start 134.870001 88.400001) (end 133.610002 89.66) (width 0.3) (layer F.Cu) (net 17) (status 20))
 (segment (start 134.4168 75.4188) (end 134.870001 75.872001) (width 0.3) (layer F.Cu) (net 17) (status 30))
 (segment (start 136.081761 85.243641) (end 135.22452 86.100882) (width 0.3) (layer F.Cu) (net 17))
 (segment (start 136.081761 77.083761) (end 136.081761 85.243641) (width 0.3) (layer F.Cu) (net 17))
 (segment (start 134.4168 75.4188) (end 136.081761 77.083761) (width 0.3) (layer F.Cu) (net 17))
 (segment (start 135.22452 88.045482) (end 134.870001 88.400001) (width 0.3) (layer F.Cu) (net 17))
 (segment (start 135.22452 86.100882) (end 135.22452 88.045482) (width 0.3) (layer F.Cu) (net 17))
 (segment (start 127.7874 77.0926) (end 126.72 78.16) (width 0.5) (layer F.Cu) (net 16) (status 20))
 (segment (start 127.7874 75.3488) (end 127.7874 77.0926) (width 0.5) (layer F.Cu) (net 16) (status 10))
 (segment (start 125.5268 77.3532) (end 124.72 78.16) (width 0.5) (layer F.Cu) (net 15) (status 20))
 (segment (start 125.5268 75.368) (end 125.5268 77.3532) (width 0.5) (layer F.Cu) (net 15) (status 10))
 (segment (start 124.477599 74.318799) (end 125.5268 75.368) (width 0.5) (layer F.Cu) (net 15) (status 20))
 (segment (start 120.825201 74.318799) (end 124.477599 74.318799) (width 0.5) (layer F.Cu) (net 15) (status 10))
 (segment (start 120.396 74.748) (end 120.825201 74.318799) (width 0.5) (layer F.Cu) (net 15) (status 30))
 (segment (start 131.39 66.5) (end 131.318 66.428) (width 0.5) (layer B.Cu) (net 2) (status 30))
 (segment (start 133.4 66.5) (end 131.39 66.5) (width 0.5) (layer B.Cu) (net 2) (status 30))
 (segment (start 131.318 67.684) (end 132.08 68.446) (width 0.5) (layer B.Cu) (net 2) (status 20))
 (segment (start 131.318 66.428) (end 131.318 67.684) (width 0.5) (layer B.Cu) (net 2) (status 10))
 (segment (start 133.52 68.446) (end 133.67 68.296) (width 0.5) (layer B.Cu) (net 2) (status 30))
 (segment (start 132.08 68.446) (end 133.52 68.446) (width 0.5) (layer B.Cu) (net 2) (status 30))
 (segment (start 131.179999 69.346001) (end 132.08 68.446) (width 0.5) (layer B.Cu) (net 2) (status 20))
 (segment (start 131.179999 71.776001) (end 131.179999 69.346001) (width 0.5) (layer B.Cu) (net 2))
 (segment (start 133.422999 73.478999) (end 131.790001 71.846001) (width 0.5) (layer B.Cu) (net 2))
 (segment (start 131.790001 71.846001) (end 131.249999 71.846001) (width 0.5) (layer B.Cu) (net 2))
 (segment (start 133.422999 73.809999) (end 133.422999 73.478999) (width 0.5) (layer B.Cu) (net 2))
 (segment (start 131.249999 71.846001) (end 131.179999 71.776001) (width 0.5) (layer B.Cu) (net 2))
 (segment (start 134.223 74.61) (end 133.422999 73.809999) (width 0.5) (layer B.Cu) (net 2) (status 10))
 (segment (start 123 62) (end 129.5 62) (width 0.5) (layer F.Cu) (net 2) (status 30))
 (segment (start 131.318 66.058002) (end 131.318 66.428) (width 0.5) (layer B.Cu) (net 2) (status 30))
 (segment (start 129.5 64.240002) (end 131.318 66.058002) (width 0.5) (layer B.Cu) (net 2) (status 20))
 (segment (start 129.5 62) (end 129.5 64.240002) (width 0.5) (layer B.Cu) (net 2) (status 10))
 (segment (start 130.048 76.832) (end 128.72 78.16) (width 0.5) (layer F.Cu) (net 14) (status 20))
 (segment (start 130.048 75.3488) (end 130.048 76.832) (width 0.5) (layer F.Cu) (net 14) (status 10))
 (segment (start 127.022 84.131) (end 126.899 84.008) (width 0.5) (layer B.Cu) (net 9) (status 30))
 (segment (start 129.794 84.131) (end 127.022 84.131) (width 0.5) (layer B.Cu) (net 9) (status 30))
 (via (at 122.682 78.232) (size 0.8) (drill 0.4) (layers F.Cu B.Cu) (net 8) (status 30))
 (segment (start 135.57 72.182) (end 135.89 72.502) (width 0.5) (layer B.Cu) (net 8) (status 20))
 (segment (start 135.57 70.896) (end 135.57 72.182) (width 0.5) (layer B.Cu) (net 8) (status 10))
 (segment (start 122.682 78.232) (end 122.682 70.866) (width 0.25) (layer B.Cu) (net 8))
 (segment (start 122.682 70.866) (end 122.809 70.739) (width 0.25) (layer B.Cu) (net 8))
 (segment (start 122.809 70.739) (end 129.109 70.739) (width 0.25) (layer B.Cu) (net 8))
 (via (at 129.109 70.739) (size 0.5) (drill 0.3) (layers F.Cu B.Cu) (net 8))
 (segment (start 129.109 70.739) (end 135.459 70.739) (width 0.25) (layer F.Cu) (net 8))
 (via (at 135.459 70.739) (size 0.5) (drill 0.3) (layers F.Cu B.Cu) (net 8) (status 30))
 (segment (start 125.1718 71.247) (end 123.4 73.0188) (width 0.5) (layer F.Cu) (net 4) (status 30))
 (segment (start 125.349 71.247) (end 125.1718 71.247) (width 0.5) (layer F.Cu) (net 4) (status 30))
 (segment (start 123.4 75.48) (end 120.72 78.16) (width 0.5) (layer F.Cu) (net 11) (status 30))
 (segment (start 123.4 75.4188) (end 123.4 75.48) (width 0.5) (layer F.Cu) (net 11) (status 30))
 (via (at 132.207 61.595) (size 0.5) (drill 0.3) (layers F.Cu B.Cu) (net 13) (status 30))
 (via (at 134.239 61.722) (size 0.5) (drill 0.3) (layers F.Cu B.Cu) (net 12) (status 30))
 (segment (start 135.636 68.23) (end 135.57 68.296) (width 0.5) (layer B.Cu) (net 12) (status 30))
 (segment (start 135.636 66.478) (end 135.636 66.548) (width 0.5) (layer B.Cu) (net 12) (status 30))
 (segment (start 135.636 66.548) (end 135.636 68.23) (width 0.5) (layer B.Cu) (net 12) (status 30))
 (via (at 135.636 66.548) (size 0.5) (drill 0.3) (layers F.Cu B.Cu) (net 12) (status 30))
 (segment (start 135.636 66.548) (end 135.636 64.262) (width 0.5) (layer F.Cu) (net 12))
 (segment (start 134.239 62.865) (end 134.239 61.722) (width 0.5) (layer F.Cu) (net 12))
 (segment (start 135.636 64.262) (end 134.239 62.865) (width 0.5) (layer F.Cu) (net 12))
 (segment (start 123 66.5) (end 129.5 66.5) (width 0.5) (layer F.Cu) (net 12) (status 30))
 (segment (start 133.55401 63.54999) (end 134.239 62.865) (width 0.5) (layer F.Cu) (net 12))
 (segment (start 132.45001 63.54999) (end 133.55401 63.54999) (width 0.5) (layer F.Cu) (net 12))
 (segment (start 129.5 66.5) (end 132.45001 63.54999) (width 0.5) (layer F.Cu) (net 12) (status 10))
 (segment (start 127.276 81.731) (end 126.899 82.108) (width 0.5) (layer B.Cu) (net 1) (status 20))
 (segment (start 129.794 81.731) (end 127.276 81.731) (width 0.5) (layer B.Cu) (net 1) (status 10))
 (segment (start 132.223 73.66) (end 133.223 74.66) (width 0.5) (layer B.Cu) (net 1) (status 10))
 (segment (start 133.223 74.66) (end 133.223 76.692616) (width 0.5) (layer B.Cu) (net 1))
 (segment (start 133.223 76.692616) (end 129.794 80.121616) (width 0.5) (layer B.Cu) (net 1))
 (segment (start 129.794 80.121616) (end 129.794 81.731) (width 0.5) (layer B.Cu) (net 1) (status 20))
 (segment (start 134.62 72.313) (end 134.223 72.71) (width 0.5) (layer B.Cu) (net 3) (status 30))
 (segment (start 134.62 70.896) (end 134.62 72.313) (width 0.5) (layer B.Cu) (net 3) (status 30))
 (segment (start 135.023001 73.510001) (end 134.223 72.71) (width 0.5) (layer B.Cu) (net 3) (status 20))
 (segment (start 130.894001 85.668997) (end 128.4765 88.086498) (width 0.5) (layer B.Cu) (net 3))
 (segment (start 135.023001 75.741157) (end 130.894001 79.870157) (width 0.5) (layer B.Cu) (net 3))
 (segment (start 130.894001 79.870157) (end 130.894001 85.668997) (width 0.5) (layer B.Cu) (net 3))
 (segment (start 128.4765 88.086498) (end 128.4765 88.5165) (width 0.5) (layer B.Cu) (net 3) (status 20))
 (segment (start 135.073001 73.560001) (end 135.023001 73.510001) (width 0.4) (layer B.Cu) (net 3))
 (segment (start 135.073001 75.691157) (end 135.073001 73.560001) (width 0.4) (layer B.Cu) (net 3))
 (segment (start 135.023001 75.741157) (end 135.073001 75.691157) (width 0.4) (layer B.Cu) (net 3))
 (segment (start 130.4765 87.5665) (end 130.5265 87.5665) (width 0.5) (layer B.Cu) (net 6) (status 30))
 (segment (start 131.494012 86.548988) (end 131.494012 81.675488) (width 0.5) (layer B.Cu) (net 6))
 (segment (start 130.4765 87.5665) (end 131.494012 86.548988) (width 0.5) (layer B.Cu) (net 6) (status 10))
 (segment (start 131.494012 81.675488) (end 133.477 79.6925) (width 0.5) (layer B.Cu) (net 6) (status 20))
 (segment (start 133.37032 79.01432) (end 134.112 78.27264) (width 0.5) (layer B.Cu) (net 6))
 (segment (start 133.37032 79.97384) (end 133.37032 79.01432) (width 0.5) (layer B.Cu) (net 6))
 (segment (start 134.08176 78.89824) (end 133.32 79.66) (width 0.5) (layer F.Cu) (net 6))
 (segment (start 134.08176 78.29804) (end 134.08176 78.89824) (width 0.5) (layer F.Cu) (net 6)))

